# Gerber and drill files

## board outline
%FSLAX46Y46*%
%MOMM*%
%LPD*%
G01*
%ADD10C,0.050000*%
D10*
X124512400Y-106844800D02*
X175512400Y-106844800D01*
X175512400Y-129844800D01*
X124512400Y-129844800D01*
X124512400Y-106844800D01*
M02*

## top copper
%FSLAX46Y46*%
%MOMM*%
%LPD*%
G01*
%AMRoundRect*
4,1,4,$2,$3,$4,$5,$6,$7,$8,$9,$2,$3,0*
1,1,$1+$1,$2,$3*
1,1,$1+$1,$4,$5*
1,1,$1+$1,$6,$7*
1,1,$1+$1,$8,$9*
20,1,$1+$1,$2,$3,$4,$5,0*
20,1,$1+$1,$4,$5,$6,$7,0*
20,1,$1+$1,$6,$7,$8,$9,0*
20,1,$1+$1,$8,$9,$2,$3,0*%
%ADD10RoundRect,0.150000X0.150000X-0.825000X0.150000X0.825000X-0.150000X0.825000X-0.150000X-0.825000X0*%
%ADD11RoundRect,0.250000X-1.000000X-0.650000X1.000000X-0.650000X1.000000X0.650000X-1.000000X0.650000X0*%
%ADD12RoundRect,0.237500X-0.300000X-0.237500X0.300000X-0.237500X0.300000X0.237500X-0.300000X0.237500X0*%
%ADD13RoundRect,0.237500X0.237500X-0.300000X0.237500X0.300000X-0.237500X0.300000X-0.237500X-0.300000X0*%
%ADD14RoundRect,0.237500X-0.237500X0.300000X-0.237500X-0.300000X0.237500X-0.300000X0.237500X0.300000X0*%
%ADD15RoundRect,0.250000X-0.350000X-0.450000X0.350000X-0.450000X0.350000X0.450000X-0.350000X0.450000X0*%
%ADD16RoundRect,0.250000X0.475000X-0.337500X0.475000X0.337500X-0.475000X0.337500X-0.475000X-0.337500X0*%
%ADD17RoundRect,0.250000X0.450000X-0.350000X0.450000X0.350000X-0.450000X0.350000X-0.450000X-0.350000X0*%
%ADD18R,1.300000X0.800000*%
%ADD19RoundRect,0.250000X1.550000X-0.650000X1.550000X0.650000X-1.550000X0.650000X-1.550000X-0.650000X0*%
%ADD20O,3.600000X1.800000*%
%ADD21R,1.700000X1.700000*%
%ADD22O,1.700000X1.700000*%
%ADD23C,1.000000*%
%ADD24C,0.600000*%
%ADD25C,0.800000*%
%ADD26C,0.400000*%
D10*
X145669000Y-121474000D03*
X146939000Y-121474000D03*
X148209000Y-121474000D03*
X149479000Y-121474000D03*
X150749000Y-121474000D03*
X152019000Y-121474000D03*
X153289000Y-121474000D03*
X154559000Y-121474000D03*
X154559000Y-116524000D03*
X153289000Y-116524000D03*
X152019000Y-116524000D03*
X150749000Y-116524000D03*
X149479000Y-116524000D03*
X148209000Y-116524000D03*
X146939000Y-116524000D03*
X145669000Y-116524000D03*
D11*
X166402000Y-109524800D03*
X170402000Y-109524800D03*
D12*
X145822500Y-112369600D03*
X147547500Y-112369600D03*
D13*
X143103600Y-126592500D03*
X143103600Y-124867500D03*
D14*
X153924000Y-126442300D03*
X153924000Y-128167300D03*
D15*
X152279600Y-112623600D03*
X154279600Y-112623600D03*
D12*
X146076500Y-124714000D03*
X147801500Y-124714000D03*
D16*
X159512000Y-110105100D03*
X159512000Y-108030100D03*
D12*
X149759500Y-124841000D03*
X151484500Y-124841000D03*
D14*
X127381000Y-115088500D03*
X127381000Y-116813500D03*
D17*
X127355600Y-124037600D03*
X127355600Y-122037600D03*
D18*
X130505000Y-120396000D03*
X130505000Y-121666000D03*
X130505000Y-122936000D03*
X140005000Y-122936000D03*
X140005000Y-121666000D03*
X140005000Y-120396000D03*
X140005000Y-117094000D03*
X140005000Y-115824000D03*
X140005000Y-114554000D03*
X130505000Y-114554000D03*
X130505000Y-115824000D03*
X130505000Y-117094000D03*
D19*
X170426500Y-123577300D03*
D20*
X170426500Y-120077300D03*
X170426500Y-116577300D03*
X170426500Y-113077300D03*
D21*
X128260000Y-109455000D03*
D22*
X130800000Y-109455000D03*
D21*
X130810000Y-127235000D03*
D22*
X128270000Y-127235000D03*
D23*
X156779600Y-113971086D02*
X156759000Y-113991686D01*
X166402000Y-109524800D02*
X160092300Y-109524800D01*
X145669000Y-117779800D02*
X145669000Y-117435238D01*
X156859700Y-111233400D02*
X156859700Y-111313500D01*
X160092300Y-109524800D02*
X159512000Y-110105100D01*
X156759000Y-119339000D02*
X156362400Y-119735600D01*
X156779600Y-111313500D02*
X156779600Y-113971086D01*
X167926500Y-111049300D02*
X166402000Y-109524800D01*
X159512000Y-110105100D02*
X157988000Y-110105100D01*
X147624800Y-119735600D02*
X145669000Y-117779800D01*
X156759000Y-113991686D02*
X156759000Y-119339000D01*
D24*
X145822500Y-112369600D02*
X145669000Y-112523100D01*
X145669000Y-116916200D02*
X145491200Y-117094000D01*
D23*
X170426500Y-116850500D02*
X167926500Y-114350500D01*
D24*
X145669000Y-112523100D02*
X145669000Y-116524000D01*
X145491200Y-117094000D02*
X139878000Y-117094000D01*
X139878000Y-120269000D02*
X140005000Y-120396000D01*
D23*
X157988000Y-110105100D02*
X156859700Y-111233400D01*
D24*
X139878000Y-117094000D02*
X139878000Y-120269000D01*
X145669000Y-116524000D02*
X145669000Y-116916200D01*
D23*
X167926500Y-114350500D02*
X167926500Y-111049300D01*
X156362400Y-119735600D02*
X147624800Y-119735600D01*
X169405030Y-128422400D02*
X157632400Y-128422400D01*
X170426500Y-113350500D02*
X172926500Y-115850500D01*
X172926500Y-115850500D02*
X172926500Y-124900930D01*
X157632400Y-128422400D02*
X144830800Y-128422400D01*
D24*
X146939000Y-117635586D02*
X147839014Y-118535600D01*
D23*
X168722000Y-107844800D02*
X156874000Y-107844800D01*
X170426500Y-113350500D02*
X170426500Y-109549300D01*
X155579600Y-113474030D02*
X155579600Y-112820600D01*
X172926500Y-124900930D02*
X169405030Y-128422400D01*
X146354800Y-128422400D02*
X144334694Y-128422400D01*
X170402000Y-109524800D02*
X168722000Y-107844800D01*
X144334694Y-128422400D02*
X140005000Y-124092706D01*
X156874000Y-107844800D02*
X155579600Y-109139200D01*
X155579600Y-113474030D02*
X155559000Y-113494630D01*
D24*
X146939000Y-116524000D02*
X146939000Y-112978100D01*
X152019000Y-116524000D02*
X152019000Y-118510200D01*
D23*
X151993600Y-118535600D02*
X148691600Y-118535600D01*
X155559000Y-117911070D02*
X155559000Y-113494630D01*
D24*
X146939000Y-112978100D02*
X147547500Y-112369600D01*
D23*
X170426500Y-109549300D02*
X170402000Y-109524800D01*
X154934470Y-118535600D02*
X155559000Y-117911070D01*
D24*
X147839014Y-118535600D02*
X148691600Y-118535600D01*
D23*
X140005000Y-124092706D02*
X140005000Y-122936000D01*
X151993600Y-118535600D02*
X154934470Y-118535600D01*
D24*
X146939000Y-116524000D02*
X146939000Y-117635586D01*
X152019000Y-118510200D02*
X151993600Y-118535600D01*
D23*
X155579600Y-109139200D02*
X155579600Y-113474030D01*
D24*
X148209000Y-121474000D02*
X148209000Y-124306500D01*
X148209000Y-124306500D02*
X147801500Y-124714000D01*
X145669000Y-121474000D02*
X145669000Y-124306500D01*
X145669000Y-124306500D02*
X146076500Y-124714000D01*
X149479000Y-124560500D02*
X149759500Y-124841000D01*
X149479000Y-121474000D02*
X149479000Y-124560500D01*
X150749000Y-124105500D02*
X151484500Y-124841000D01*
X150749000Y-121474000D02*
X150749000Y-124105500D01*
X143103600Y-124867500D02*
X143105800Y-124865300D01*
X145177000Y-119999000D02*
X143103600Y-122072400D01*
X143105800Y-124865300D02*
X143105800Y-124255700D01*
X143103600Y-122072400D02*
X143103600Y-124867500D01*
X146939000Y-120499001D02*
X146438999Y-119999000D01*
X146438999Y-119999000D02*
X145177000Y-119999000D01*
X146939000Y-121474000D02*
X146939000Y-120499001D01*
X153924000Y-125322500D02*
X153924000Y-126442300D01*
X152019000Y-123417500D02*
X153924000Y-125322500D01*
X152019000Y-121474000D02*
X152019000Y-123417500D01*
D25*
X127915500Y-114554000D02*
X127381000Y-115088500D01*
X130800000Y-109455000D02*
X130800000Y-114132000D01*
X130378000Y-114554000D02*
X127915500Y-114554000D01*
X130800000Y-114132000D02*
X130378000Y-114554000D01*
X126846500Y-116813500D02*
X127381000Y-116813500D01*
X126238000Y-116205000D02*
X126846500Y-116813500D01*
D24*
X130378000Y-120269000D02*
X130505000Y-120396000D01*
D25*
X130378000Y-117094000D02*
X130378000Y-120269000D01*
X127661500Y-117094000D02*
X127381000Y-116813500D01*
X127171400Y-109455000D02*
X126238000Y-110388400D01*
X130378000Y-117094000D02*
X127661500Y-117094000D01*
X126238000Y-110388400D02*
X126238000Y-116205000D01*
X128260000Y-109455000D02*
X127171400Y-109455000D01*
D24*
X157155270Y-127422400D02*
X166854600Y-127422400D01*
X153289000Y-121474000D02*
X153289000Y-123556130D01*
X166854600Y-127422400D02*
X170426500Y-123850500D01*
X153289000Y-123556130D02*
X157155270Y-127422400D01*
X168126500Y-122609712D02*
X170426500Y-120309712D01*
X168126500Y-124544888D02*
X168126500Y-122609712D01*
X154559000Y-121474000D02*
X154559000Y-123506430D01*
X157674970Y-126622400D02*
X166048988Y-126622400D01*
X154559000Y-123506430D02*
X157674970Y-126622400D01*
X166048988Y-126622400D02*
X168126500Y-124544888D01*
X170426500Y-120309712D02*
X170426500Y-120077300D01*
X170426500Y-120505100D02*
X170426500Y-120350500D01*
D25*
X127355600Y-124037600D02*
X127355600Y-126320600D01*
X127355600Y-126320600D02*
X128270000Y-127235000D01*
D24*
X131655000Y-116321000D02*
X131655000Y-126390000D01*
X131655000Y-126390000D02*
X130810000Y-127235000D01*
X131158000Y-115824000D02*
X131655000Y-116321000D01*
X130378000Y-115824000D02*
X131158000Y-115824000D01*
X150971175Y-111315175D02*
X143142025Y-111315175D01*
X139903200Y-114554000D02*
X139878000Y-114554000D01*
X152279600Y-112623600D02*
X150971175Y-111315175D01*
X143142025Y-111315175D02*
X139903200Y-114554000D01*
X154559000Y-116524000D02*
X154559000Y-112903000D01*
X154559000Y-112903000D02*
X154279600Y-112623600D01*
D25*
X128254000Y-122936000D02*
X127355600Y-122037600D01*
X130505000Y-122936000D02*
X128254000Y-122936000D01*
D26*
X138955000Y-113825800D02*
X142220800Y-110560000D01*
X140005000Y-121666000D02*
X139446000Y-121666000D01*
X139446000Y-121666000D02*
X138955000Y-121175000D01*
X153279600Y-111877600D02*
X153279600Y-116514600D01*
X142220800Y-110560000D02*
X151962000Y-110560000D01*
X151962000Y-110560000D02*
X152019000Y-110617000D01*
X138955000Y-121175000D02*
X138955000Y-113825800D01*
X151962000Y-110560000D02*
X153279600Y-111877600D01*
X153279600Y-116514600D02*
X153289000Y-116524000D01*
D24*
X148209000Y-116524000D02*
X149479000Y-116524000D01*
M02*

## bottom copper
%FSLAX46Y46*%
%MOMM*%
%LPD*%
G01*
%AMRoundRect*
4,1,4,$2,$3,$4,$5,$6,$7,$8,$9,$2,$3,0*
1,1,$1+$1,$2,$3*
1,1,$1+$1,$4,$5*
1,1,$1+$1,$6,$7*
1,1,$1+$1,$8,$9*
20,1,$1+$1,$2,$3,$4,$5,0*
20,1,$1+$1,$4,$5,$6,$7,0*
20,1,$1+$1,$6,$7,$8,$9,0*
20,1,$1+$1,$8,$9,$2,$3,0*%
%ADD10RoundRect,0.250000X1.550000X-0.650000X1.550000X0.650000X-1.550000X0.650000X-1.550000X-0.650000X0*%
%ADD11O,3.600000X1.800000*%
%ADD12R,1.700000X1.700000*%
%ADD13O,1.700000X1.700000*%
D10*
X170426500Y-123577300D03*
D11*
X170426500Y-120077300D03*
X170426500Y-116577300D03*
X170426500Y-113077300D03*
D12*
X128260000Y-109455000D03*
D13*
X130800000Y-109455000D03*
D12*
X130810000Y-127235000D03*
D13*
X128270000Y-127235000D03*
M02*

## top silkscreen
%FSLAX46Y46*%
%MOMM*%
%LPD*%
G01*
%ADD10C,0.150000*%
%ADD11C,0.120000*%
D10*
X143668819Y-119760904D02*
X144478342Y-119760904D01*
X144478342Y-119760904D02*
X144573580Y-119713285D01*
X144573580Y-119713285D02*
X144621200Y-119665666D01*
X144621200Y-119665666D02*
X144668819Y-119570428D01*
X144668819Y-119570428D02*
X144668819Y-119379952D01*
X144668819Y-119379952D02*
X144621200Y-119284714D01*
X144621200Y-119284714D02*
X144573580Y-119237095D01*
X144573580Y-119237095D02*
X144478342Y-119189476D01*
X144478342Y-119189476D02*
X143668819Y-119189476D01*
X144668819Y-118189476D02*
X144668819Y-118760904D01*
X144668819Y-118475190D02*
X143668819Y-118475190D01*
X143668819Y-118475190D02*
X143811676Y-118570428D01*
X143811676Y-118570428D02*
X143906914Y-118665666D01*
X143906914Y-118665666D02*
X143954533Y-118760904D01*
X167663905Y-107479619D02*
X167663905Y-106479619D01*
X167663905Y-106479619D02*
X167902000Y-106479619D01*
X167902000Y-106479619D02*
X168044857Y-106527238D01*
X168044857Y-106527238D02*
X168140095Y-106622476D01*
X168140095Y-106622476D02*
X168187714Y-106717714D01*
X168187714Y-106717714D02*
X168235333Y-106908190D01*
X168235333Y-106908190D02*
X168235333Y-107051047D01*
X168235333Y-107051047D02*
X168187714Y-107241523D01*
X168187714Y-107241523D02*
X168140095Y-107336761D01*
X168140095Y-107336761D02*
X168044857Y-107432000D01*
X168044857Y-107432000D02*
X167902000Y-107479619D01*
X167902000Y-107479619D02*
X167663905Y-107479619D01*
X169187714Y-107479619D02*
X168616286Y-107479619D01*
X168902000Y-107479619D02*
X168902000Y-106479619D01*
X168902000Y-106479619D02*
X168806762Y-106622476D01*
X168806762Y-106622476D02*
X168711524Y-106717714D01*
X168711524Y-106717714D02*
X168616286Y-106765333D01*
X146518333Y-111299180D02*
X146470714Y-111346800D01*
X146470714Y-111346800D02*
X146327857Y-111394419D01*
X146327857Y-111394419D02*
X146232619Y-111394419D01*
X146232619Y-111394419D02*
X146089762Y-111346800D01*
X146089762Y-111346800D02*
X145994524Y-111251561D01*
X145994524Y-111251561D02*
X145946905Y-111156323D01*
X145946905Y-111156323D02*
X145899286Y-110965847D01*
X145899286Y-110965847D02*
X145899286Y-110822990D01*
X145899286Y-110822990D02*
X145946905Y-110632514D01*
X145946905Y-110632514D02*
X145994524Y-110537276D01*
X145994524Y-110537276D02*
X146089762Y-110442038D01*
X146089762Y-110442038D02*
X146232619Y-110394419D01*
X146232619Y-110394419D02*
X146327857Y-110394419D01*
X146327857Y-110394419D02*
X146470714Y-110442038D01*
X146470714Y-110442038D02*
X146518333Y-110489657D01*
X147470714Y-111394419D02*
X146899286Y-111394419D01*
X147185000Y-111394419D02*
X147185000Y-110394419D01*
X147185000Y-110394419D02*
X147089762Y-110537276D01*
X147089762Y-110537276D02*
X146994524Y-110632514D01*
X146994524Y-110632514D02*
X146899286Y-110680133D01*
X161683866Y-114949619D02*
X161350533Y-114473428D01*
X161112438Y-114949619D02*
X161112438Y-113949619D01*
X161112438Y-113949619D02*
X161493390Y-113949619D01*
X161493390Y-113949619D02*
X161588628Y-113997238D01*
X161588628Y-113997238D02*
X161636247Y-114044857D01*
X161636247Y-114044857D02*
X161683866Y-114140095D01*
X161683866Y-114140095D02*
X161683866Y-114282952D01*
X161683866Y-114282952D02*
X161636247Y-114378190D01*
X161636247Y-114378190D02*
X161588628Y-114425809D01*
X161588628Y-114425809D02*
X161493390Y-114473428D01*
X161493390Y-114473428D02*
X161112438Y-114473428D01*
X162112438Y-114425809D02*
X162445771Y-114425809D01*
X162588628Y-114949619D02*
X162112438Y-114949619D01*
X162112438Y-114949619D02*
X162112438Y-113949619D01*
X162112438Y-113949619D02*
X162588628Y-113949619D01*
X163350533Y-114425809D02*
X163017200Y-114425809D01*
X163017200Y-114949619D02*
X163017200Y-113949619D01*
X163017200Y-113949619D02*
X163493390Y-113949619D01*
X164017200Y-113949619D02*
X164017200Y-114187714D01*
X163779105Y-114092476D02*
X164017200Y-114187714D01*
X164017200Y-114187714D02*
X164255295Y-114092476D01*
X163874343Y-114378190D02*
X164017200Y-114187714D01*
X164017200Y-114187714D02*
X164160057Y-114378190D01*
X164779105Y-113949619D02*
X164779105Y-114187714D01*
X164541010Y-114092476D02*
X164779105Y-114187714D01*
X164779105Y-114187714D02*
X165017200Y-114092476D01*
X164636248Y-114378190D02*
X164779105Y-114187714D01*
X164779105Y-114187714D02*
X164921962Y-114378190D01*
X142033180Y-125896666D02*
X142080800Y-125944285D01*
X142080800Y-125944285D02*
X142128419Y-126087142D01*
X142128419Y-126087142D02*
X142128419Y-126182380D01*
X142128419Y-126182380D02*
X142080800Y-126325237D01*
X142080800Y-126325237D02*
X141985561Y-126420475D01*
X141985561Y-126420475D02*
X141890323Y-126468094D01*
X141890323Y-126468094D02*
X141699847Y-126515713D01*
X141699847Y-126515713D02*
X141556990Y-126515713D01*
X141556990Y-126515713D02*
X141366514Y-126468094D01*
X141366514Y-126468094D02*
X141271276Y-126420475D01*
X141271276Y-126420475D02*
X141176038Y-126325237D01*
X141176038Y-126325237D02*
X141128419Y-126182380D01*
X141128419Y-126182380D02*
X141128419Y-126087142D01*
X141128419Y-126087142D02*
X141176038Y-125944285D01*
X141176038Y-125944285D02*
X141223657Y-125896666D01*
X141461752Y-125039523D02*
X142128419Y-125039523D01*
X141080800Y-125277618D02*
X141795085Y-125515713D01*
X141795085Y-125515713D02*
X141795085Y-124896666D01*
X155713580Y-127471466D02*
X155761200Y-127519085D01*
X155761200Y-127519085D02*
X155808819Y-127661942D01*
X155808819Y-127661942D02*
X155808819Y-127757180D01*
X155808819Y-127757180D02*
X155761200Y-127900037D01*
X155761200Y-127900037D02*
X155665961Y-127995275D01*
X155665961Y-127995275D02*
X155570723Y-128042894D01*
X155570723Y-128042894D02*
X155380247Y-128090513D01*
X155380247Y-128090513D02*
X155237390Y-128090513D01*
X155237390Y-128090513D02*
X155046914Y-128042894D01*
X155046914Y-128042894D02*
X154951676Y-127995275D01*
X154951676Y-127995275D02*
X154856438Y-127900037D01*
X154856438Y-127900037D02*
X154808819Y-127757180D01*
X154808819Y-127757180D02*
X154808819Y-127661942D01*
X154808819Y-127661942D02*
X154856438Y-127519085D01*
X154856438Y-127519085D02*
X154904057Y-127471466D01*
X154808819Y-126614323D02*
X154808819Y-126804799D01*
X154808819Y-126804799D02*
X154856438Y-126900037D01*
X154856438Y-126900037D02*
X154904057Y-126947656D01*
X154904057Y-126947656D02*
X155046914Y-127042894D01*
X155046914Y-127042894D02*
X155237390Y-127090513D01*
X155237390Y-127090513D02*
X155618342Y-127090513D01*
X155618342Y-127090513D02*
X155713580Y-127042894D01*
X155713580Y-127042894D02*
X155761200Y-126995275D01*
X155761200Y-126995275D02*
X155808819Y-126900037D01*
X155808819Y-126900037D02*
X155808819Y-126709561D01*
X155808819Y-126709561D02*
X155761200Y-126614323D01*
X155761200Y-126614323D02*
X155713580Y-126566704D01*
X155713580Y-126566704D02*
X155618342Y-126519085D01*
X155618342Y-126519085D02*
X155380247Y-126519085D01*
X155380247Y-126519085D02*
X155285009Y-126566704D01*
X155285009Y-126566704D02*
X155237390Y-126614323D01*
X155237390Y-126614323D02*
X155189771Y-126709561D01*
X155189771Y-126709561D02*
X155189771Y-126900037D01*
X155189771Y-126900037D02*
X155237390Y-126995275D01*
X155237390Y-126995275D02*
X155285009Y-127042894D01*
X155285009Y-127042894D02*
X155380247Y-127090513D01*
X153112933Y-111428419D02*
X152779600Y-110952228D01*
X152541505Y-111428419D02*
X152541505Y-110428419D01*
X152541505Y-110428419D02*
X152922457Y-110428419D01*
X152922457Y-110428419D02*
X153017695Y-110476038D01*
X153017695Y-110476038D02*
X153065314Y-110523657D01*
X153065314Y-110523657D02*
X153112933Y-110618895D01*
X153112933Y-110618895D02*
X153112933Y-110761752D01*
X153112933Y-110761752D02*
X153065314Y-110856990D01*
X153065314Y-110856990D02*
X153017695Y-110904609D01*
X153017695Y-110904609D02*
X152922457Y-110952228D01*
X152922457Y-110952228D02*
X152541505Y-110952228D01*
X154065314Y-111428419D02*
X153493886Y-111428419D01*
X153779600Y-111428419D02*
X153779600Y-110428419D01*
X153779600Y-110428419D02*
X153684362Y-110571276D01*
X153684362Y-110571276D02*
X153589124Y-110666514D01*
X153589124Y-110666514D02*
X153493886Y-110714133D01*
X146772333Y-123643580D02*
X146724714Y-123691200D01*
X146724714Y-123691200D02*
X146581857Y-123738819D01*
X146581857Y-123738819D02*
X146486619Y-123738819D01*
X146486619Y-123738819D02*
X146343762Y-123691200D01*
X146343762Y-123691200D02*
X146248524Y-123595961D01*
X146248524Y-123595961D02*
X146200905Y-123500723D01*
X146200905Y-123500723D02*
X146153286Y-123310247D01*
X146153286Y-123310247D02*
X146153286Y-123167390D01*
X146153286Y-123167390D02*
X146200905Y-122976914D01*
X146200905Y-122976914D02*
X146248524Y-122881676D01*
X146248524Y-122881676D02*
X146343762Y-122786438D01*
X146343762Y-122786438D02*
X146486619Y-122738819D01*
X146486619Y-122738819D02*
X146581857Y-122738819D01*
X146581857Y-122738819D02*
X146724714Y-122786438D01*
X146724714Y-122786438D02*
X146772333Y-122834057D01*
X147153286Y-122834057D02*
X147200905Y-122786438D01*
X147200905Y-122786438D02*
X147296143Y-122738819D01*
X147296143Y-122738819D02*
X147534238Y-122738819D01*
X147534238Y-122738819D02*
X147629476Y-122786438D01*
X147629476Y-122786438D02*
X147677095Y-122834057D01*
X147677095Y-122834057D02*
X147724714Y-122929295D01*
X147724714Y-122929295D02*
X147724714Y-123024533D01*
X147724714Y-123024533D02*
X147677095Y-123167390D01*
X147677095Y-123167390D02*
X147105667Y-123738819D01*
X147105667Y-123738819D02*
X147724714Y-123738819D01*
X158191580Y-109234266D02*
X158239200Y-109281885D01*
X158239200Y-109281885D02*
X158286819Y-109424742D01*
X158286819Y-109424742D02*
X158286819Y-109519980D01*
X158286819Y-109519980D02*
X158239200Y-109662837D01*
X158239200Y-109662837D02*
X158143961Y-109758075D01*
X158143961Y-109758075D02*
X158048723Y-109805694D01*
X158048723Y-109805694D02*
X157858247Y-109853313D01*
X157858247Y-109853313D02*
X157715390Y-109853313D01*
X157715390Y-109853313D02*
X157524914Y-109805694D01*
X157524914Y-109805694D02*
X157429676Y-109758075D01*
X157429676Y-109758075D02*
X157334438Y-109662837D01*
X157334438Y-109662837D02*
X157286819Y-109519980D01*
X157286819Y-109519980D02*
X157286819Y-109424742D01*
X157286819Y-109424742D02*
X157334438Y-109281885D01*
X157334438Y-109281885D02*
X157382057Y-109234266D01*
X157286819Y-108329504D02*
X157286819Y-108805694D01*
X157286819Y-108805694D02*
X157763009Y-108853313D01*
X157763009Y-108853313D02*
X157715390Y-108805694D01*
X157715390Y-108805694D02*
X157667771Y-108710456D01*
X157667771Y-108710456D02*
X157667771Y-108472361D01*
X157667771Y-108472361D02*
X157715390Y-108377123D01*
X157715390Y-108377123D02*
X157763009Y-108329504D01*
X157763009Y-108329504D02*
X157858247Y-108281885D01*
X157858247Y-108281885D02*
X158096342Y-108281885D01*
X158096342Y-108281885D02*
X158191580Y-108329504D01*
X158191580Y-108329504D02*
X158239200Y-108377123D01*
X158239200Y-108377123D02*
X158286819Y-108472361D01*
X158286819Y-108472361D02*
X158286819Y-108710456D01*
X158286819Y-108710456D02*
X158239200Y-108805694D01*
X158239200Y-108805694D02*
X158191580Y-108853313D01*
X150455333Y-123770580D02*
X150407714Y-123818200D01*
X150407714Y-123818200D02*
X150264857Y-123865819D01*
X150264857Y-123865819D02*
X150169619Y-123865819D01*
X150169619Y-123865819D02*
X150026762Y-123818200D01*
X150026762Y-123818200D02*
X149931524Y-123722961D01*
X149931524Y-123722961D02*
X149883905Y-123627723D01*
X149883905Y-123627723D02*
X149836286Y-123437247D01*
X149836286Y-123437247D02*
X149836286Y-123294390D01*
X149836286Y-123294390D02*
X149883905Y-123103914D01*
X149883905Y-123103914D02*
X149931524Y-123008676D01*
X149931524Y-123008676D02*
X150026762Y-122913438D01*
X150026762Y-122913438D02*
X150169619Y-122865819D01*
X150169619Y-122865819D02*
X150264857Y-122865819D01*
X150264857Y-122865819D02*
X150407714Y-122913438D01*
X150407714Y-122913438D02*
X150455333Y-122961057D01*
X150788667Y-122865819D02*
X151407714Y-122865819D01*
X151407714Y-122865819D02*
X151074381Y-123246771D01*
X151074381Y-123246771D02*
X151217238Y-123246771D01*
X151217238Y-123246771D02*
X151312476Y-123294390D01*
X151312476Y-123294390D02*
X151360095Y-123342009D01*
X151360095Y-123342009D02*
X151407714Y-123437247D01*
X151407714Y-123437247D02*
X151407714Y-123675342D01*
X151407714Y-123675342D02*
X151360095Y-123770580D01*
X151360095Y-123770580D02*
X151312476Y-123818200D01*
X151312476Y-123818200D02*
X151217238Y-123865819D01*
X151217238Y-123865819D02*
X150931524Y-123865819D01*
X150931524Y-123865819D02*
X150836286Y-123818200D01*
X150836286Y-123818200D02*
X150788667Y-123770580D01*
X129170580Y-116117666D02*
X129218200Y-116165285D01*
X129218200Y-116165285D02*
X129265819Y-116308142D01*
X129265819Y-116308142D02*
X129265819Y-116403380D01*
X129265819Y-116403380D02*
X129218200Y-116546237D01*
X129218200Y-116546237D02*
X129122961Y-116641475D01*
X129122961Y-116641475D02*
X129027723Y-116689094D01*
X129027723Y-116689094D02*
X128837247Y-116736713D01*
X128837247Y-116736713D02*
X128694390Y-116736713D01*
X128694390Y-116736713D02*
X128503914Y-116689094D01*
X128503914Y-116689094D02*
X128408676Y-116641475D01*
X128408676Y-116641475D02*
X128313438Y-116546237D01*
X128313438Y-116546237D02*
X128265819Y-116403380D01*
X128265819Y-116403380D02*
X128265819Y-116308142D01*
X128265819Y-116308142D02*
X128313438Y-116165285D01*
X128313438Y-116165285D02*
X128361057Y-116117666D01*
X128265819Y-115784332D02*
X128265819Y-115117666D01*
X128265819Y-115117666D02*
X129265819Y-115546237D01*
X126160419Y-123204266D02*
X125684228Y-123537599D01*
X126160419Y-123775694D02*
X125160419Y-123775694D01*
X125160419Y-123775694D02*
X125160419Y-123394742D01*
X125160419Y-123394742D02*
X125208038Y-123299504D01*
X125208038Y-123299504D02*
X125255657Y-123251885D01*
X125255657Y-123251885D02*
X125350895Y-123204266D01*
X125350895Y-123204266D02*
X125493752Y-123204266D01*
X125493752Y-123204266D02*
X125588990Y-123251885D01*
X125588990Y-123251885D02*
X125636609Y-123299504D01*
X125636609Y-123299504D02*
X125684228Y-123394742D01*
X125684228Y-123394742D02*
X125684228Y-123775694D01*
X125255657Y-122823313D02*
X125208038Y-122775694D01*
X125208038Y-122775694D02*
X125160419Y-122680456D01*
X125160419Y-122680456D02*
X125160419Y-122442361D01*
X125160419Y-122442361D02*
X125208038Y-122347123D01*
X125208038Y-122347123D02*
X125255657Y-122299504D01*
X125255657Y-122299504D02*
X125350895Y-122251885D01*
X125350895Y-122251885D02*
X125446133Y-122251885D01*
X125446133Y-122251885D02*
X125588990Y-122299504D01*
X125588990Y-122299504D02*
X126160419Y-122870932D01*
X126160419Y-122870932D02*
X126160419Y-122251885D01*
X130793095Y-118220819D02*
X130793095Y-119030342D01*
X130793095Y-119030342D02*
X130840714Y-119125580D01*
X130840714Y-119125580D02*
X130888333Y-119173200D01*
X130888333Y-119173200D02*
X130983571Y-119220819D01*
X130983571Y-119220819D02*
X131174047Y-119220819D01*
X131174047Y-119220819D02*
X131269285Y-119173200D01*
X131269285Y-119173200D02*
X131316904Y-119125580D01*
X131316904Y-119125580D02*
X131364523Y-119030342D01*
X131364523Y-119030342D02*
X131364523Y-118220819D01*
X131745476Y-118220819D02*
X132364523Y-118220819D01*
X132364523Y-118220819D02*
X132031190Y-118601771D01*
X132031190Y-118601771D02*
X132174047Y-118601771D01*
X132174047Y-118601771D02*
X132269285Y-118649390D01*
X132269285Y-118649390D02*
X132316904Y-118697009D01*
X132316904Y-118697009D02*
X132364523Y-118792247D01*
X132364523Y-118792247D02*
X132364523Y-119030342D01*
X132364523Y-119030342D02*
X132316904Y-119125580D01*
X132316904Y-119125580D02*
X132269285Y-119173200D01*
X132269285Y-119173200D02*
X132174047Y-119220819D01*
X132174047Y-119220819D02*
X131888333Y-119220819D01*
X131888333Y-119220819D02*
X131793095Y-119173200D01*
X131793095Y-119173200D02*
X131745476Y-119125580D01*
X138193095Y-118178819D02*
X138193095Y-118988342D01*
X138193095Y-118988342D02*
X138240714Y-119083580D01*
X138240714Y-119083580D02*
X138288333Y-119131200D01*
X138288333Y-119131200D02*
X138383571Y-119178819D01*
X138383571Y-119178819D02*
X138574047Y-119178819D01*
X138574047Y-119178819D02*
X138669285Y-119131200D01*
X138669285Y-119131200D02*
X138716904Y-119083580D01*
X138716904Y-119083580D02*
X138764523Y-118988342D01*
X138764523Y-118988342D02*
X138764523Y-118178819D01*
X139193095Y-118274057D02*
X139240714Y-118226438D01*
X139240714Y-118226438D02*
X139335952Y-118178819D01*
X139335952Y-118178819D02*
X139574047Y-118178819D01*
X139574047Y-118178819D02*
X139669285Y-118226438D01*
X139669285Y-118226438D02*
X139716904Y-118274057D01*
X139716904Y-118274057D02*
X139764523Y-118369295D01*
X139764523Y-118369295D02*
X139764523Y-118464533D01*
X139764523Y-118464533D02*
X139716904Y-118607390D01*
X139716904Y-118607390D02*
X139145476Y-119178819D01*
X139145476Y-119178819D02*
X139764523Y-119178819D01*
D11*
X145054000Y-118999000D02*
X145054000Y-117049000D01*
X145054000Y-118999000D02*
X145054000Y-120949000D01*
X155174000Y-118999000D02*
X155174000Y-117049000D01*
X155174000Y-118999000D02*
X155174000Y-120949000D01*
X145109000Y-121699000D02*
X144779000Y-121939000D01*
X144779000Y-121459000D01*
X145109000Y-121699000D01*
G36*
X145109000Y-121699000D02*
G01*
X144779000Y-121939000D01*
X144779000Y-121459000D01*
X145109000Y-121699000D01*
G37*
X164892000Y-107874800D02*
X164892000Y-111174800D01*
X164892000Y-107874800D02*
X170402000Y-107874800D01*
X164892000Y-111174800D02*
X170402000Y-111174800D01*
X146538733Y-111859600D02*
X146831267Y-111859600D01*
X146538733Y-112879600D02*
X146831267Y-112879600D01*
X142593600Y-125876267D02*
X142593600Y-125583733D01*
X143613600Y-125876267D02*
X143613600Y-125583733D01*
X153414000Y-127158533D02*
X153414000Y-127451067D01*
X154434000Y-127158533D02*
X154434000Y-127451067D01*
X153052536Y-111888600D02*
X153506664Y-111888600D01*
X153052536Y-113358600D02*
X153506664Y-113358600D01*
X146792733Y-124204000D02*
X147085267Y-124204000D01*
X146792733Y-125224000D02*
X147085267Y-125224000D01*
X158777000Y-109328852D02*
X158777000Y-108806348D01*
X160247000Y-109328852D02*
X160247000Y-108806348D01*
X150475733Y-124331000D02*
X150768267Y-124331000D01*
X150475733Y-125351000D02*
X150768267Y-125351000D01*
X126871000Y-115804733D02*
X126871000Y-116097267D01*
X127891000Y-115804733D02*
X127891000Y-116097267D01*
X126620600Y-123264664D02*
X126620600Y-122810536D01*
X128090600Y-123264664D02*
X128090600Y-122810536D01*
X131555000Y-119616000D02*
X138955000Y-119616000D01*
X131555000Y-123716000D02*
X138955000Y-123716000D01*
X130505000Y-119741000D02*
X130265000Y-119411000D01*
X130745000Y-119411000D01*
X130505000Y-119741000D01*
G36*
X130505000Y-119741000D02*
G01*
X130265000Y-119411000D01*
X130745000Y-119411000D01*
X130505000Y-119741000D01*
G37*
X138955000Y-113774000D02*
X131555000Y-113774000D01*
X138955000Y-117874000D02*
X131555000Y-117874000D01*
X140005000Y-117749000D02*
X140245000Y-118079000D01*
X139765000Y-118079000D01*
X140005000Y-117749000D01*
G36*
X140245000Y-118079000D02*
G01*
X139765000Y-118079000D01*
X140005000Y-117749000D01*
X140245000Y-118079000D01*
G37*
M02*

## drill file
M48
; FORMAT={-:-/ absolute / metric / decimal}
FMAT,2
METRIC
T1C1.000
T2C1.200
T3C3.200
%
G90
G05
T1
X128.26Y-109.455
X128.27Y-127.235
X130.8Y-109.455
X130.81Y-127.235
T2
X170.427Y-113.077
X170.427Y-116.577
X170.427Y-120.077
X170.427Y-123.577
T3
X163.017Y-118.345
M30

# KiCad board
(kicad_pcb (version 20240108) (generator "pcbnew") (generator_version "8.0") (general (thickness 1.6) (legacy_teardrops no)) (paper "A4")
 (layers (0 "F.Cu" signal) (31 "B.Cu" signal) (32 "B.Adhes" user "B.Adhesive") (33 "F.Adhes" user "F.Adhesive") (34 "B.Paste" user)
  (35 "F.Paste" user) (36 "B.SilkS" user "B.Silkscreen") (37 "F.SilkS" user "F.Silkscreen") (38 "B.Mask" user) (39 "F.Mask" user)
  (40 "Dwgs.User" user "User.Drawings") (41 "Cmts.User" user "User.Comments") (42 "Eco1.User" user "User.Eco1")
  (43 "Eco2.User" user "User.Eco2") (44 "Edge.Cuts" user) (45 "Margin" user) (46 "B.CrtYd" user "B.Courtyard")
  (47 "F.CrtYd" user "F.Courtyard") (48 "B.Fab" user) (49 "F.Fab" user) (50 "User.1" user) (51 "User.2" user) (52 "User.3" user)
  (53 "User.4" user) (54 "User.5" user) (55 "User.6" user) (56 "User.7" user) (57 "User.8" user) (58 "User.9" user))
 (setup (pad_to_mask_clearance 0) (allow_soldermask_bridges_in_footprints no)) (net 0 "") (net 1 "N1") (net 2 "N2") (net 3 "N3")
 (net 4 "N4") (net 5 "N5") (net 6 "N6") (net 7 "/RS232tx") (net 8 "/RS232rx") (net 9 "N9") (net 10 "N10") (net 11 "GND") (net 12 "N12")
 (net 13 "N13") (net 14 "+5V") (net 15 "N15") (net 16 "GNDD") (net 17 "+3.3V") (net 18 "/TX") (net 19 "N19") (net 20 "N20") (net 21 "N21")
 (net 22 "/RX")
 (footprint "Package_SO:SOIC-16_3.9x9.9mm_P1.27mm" (layer "F.Cu") (at 150.114 118.999 90)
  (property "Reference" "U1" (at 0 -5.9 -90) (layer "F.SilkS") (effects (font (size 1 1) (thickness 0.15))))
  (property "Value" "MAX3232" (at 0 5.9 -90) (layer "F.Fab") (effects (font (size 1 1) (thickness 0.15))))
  (fp_line (start 0 -5.06) (end 1.95 -5.06) (stroke (width 0.12) (type solid)) (layer "F.SilkS"))
  (fp_line (start 0 -5.06) (end -1.95 -5.06) (stroke (width 0.12) (type solid)) (layer "F.SilkS"))
  (fp_line (start 0 5.06) (end 1.95 5.06) (stroke (width 0.12) (type solid)) (layer "F.SilkS"))
  (fp_line (start 0 5.06) (end -1.95 5.06) (stroke (width 0.12) (type solid)) (layer "F.SilkS"))
  (fp_poly
   (pts (xy -2.7 -5.005) (xy -2.94 -5.335) (xy -2.46 -5.335) (xy -2.7 -5.005)) (stroke (width 0.12) (type solid)) (fill solid)
   (layer "F.SilkS"))
  (pad "1" smd roundrect (at -2.475 -4.445 90) (size 1.95 0.6) (layers "F.Cu" "F.Paste" "F.Mask") (roundrect_rratio 0.25) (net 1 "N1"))
  (pad "2" smd roundrect (at -2.475 -3.175 90) (size 1.95 0.6) (layers "F.Cu" "F.Paste" "F.Mask") (roundrect_rratio 0.25) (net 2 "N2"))
  (pad "3" smd roundrect (at -2.475 -1.905 90) (size 1.95 0.6) (layers "F.Cu" "F.Paste" "F.Mask") (roundrect_rratio 0.25) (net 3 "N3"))
  (pad "4" smd roundrect (at -2.475 -0.635 90) (size 1.95 0.6) (layers "F.Cu" "F.Paste" "F.Mask") (roundrect_rratio 0.25) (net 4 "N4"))
  (pad "5" smd roundrect (at -2.475 0.635 90) (size 1.95 0.6) (layers "F.Cu" "F.Paste" "F.Mask") (roundrect_rratio 0.25) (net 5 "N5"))
  (pad "6" smd roundrect (at -2.475 1.905 90) (size 1.95 0.6) (layers "F.Cu" "F.Paste" "F.Mask") (roundrect_rratio 0.25) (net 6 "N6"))
  (pad "7" smd roundrect (at -2.475 3.175 90) (size 1.95 0.6) (layers "F.Cu" "F.Paste" "F.Mask") (roundrect_rratio 0.25) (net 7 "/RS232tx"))
  (pad "8" smd roundrect (at -2.475 4.445 90) (size 1.95 0.6) (layers "F.Cu" "F.Paste" "F.Mask") (roundrect_rratio 0.25) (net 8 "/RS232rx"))
  (pad "9" smd roundrect (at 2.475 4.445 90) (size 1.95 0.6) (layers "F.Cu" "F.Paste" "F.Mask") (roundrect_rratio 0.25) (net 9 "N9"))
  (pad "10" smd roundrect (at 2.475 3.175 90) (size 1.95 0.6) (layers "F.Cu" "F.Paste" "F.Mask") (roundrect_rratio 0.25) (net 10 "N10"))
  (pad "11" smd roundrect (at 2.475 1.905 90) (size 1.95 0.6) (layers "F.Cu" "F.Paste" "F.Mask") (roundrect_rratio 0.25) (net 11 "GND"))
  (pad "12" smd roundrect (at 2.475 0.635 90) (size 1.95 0.6) (layers "F.Cu" "F.Paste" "F.Mask") (roundrect_rratio 0.25) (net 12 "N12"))
  (pad "13" smd roundrect (at 2.475 -0.635 90) (size 1.95 0.6) (layers "F.Cu" "F.Paste" "F.Mask") (roundrect_rratio 0.25) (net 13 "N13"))
  (pad "14" smd roundrect (at 2.475 -1.905 90) (size 1.95 0.6) (layers "F.Cu" "F.Paste" "F.Mask") (roundrect_rratio 0.25) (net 13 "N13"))
  (pad "15" smd roundrect (at 2.475 -3.175 90) (size 1.95 0.6) (layers "F.Cu" "F.Paste" "F.Mask") (roundrect_rratio 0.25) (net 11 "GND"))
  (pad "16" smd roundrect (at 2.475 -4.445 90) (size 1.95 0.6) (layers "F.Cu" "F.Paste" "F.Mask") (roundrect_rratio 0.25) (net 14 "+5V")))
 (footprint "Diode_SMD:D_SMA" (layer "F.Cu") (at 168.402 109.5248)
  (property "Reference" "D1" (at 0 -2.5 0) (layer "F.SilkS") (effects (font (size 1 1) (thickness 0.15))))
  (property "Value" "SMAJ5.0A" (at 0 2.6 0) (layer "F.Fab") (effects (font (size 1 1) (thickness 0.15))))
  (fp_line (start -3.51 -1.65) (end -3.51 1.65) (stroke (width 0.12) (type solid)) (layer "F.SilkS"))
  (fp_line (start -3.51 -1.65) (end 2 -1.65) (stroke (width 0.12) (type solid)) (layer "F.SilkS"))
  (fp_line (start -3.51 1.65) (end 2 1.65) (stroke (width 0.12) (type solid)) (layer "F.SilkS"))
  (pad "1" smd roundrect (at -2 0) (size 2.5 1.8) (layers "F.Cu" "F.Paste" "F.Mask") (roundrect_rratio 0.1388888889) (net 14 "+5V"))
  (pad "2" smd roundrect (at 2 0) (size 2.5 1.8) (layers "F.Cu" "F.Paste" "F.Mask") (roundrect_rratio 0.1388888889) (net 11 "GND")))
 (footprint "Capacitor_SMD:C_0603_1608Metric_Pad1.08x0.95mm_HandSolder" (layer "F.Cu") (at 146.685 112.3696)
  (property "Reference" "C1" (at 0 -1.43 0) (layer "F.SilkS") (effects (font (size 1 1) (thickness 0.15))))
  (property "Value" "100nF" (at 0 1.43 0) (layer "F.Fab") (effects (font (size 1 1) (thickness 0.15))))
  (fp_line (start -0.146267 -0.51) (end 0.146267 -0.51) (stroke (width 0.12) (type solid)) (layer "F.SilkS"))
  (fp_line (start -0.146267 0.51) (end 0.146267 0.51) (stroke (width 0.12) (type solid)) (layer "F.SilkS"))
  (pad "1" smd roundrect (at -0.8625 0) (size 1.075 0.95) (layers "F.Cu" "F.Paste" "F.Mask") (roundrect_rratio 0.25) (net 14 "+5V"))
  (pad "2" smd roundrect (at 0.8625 0) (size 1.075 0.95) (layers "F.Cu" "F.Paste" "F.Mask") (roundrect_rratio 0.25) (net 11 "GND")))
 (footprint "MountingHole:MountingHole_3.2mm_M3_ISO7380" (layer "F.Cu") (at 163.0172 118.3448)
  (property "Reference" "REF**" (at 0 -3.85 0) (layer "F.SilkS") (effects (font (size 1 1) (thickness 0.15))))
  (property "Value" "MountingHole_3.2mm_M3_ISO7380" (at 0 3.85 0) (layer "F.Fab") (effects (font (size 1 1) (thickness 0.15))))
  (pad "" np_thru_hole circle (at 0 0) (size 3.2 3.2) (drill 3.2) (layers "F&B.Cu" "*.Mask") (clearance 4)))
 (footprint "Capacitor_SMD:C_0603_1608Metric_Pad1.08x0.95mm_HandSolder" (layer "F.Cu") (at 143.1036 125.73 90)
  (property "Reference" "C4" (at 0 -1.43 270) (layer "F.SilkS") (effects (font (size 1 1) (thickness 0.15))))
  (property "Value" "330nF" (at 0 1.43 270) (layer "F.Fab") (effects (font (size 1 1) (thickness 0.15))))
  (fp_line (start -0.146267 -0.51) (end 0.146267 -0.51) (stroke (width 0.12) (type solid)) (layer "F.SilkS"))
  (fp_line (start -0.146267 0.51) (end 0.146267 0.51) (stroke (width 0.12) (type solid)) (layer "F.SilkS"))
  (pad "1" smd roundrect (at -0.8625 0 90) (size 1.075 0.95) (layers "F.Cu" "F.Paste" "F.Mask") (roundrect_rratio 0.25) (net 11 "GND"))
  (pad "2" smd roundrect (at 0.8625 0 90) (size 1.075 0.95) (layers "F.Cu" "F.Paste" "F.Mask") (roundrect_rratio 0.25) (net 2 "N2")))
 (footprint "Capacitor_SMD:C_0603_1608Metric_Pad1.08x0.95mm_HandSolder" (layer "F.Cu") (at 153.924 127.3048 -90)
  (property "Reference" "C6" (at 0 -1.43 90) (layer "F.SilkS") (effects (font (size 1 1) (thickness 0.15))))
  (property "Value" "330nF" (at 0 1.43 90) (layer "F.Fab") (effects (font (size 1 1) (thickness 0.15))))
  (fp_line (start -0.146267 0.51) (end 0.146267 0.51) (stroke (width 0.12) (type solid)) (layer "F.SilkS"))
  (fp_line (start -0.146267 -0.51) (end 0.146267 -0.51) (stroke (width 0.12) (type solid)) (layer "F.SilkS"))
  (pad "1" smd roundrect (at -0.8625 0 270) (size 1.075 0.95) (layers "F.Cu" "F.Paste" "F.Mask") (roundrect_rratio 0.25) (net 6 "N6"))
  (pad "2" smd roundrect (at 0.8625 0 270) (size 1.075 0.95) (layers "F.Cu" "F.Paste" "F.Mask") (roundrect_rratio 0.25) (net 11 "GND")))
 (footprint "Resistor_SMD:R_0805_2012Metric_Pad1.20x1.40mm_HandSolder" (layer "F.Cu") (at 153.2796 112.6236)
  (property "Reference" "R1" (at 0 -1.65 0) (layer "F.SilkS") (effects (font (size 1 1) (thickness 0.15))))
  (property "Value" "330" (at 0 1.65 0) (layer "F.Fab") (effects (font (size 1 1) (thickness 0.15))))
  (fp_line (start -0.227064 -0.735) (end 0.227064 -0.735) (stroke (width 0.12) (type solid)) (layer "F.SilkS"))
  (fp_line (start -0.227064 0.735) (end 0.227064 0.735) (stroke (width 0.12) (type solid)) (layer "F.SilkS"))
  (pad "1" smd roundrect (at -1 0) (size 1.2 1.4) (layers "F.Cu" "F.Paste" "F.Mask") (roundrect_rratio 0.208333) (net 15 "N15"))
  (pad "2" smd roundrect (at 1 0) (size 1.2 1.4) (layers "F.Cu" "F.Paste" "F.Mask") (roundrect_rratio 0.208333) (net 9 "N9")))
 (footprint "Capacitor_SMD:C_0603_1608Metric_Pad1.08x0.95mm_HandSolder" (layer "F.Cu") (at 146.939 124.714)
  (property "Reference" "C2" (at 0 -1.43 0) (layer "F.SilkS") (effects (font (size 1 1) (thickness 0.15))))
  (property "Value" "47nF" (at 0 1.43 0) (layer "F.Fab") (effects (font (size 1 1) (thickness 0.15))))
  (fp_line (start -0.146267 -0.51) (end 0.146267 -0.51) (stroke (width 0.12) (type solid)) (layer "F.SilkS"))
  (fp_line (start -0.146267 0.51) (end 0.146267 0.51) (stroke (width 0.12) (type solid)) (layer "F.SilkS"))
  (pad "1" smd roundrect (at -0.8625 0) (size 1.075 0.95) (layers "F.Cu" "F.Paste" "F.Mask") (roundrect_rratio 0.25) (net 1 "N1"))
  (pad "2" smd roundrect (at 0.8625 0) (size 1.075 0.95) (layers "F.Cu" "F.Paste" "F.Mask") (roundrect_rratio 0.25) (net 3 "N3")))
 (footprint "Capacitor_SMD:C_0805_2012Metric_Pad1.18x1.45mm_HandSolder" (layer "F.Cu") (at 159.512 109.0676 90)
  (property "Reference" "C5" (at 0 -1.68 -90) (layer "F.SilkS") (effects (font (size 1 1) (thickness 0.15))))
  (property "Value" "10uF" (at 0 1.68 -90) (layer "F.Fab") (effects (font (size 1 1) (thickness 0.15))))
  (fp_line (start -0.261252 -0.735) (end 0.261252 -0.735) (stroke (width 0.12) (type solid)) (layer "F.SilkS"))
  (fp_line (start -0.261252 0.735) (end 0.261252 0.735) (stroke (width 0.12) (type solid)) (layer "F.SilkS"))
  (pad "1" smd roundrect (at -1.0375 0 90) (size 1.175 1.45) (layers "F.Cu" "F.Paste" "F.Mask") (roundrect_rratio 0.212766) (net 14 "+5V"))
  (pad "2" smd roundrect (at 1.0375 0 90) (size 1.175 1.45) (layers "F.Cu" "F.Paste" "F.Mask") (roundrect_rratio 0.212766) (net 11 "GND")))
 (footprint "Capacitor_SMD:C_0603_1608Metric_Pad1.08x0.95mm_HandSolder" (layer "F.Cu") (at 150.622 124.841)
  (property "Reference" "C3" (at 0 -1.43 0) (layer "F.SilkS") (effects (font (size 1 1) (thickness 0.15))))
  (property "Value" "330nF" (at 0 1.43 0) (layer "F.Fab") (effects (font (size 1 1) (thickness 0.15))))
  (fp_line (start -0.146267 -0.51) (end 0.146267 -0.51) (stroke (width 0.12) (type solid)) (layer "F.SilkS"))
  (fp_line (start -0.146267 0.51) (end 0.146267 0.51) (stroke (width 0.12) (type solid)) (layer "F.SilkS"))
  (pad "1" smd roundrect (at -0.8625 0) (size 1.075 0.95) (layers "F.Cu" "F.Paste" "F.Mask") (roundrect_rratio 0.25) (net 4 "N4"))
  (pad "2" smd roundrect (at 0.8625 0) (size 1.075 0.95) (layers "F.Cu" "F.Paste" "F.Mask") (roundrect_rratio 0.25) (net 5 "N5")))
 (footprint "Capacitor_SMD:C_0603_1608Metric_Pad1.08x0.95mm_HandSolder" (layer "F.Cu") (at 127.381 115.951 -90)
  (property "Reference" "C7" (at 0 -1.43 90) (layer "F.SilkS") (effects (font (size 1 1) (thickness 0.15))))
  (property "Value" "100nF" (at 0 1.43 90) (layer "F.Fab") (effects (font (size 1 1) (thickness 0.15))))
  (fp_line (start -0.146267 0.51) (end 0.146267 0.51) (stroke (width 0.12) (type solid)) (layer "F.SilkS"))
  (fp_line (start -0.146267 -0.51) (end 0.146267 -0.51) (stroke (width 0.12) (type solid)) (layer "F.SilkS"))
  (pad "1" smd roundrect (at -0.8625 0 270) (size 1.075 0.95) (layers "F.Cu" "F.Paste" "F.Mask") (roundrect_rratio 0.25) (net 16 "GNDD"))
  (pad "2" smd roundrect (at 0.8625 0 270) (size 1.075 0.95) (layers "F.Cu" "F.Paste" "F.Mask") (roundrect_rratio 0.25) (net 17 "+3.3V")))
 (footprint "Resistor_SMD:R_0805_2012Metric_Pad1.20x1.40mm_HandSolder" (layer "F.Cu") (at 127.3556 123.0376 90)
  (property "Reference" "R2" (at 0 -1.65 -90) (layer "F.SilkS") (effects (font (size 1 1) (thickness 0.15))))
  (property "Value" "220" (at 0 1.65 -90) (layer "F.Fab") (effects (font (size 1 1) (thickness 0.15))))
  (fp_line (start -0.227064 -0.735) (end 0.227064 -0.735) (stroke (width 0.12) (type solid)) (layer "F.SilkS"))
  (fp_line (start -0.227064 0.735) (end 0.227064 0.735) (stroke (width 0.12) (type solid)) (layer "F.SilkS"))
  (pad "1" smd roundrect (at -1 0 90) (size 1.2 1.4) (layers "F.Cu" "F.Paste" "F.Mask") (roundrect_rratio 0.208333) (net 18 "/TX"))
  (pad "2" smd roundrect (at 1 0 90) (size 1.2 1.4) (layers "F.Cu" "F.Paste" "F.Mask") (roundrect_rratio 0.208333) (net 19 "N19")))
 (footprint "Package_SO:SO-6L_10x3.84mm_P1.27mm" (layer "F.Cu") (at 135.255 121.666)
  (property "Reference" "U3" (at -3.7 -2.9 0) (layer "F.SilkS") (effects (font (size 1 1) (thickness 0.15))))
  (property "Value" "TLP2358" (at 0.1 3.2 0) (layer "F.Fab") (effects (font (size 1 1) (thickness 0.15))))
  (fp_line (start -3.7 -2.05) (end 3.7 -2.05) (stroke (width 0.12) (type solid)) (layer "F.SilkS"))
  (fp_line (start -3.7 2.05) (end 3.7 2.05) (stroke (width 0.12) (type solid)) (layer "F.SilkS"))
  (fp_poly
   (pts (xy -4.75 -1.925) (xy -4.99 -2.255) (xy -4.51 -2.255) (xy -4.75 -1.925)) (stroke (width 0.12) (type solid)) (fill solid)
   (layer "F.SilkS"))
  (pad "1" smd rect (at -4.75 -1.27 90) (size 0.8 1.3) (layers "F.Cu" "F.Paste" "F.Mask") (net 17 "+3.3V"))
  (pad "2" smd rect (at -4.75 0 90) (size 0.8 1.3) (layers "F.Cu" "F.Paste" "F.Mask") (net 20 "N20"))
  (pad "3" smd rect (at -4.75 1.27 90) (size 0.8 1.3) (layers "F.Cu" "F.Paste" "F.Mask") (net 19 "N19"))
  (pad "4" smd rect (at 4.75 1.27 90) (size 0.8 1.3) (layers "F.Cu" "F.Paste" "F.Mask") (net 11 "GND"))
  (pad "5" smd rect (at 4.75 0 90) (size 0.8 1.3) (layers "F.Cu" "F.Paste" "F.Mask") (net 10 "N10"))
  (pad "6" smd rect (at 4.75 -1.27 90) (size 0.8 1.3) (layers "F.Cu" "F.Paste" "F.Mask") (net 14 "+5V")))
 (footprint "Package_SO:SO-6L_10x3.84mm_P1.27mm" (layer "F.Cu") (at 135.255 115.824 180)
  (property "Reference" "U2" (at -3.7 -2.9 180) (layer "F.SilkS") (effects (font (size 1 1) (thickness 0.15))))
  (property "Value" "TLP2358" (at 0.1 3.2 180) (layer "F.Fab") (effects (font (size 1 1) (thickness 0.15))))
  (fp_line (start -3.7 2.05) (end 3.7 2.05) (stroke (width 0.12) (type solid)) (layer "F.SilkS"))
  (fp_line (start -3.7 -2.05) (end 3.7 -2.05) (stroke (width 0.12) (type solid)) (layer "F.SilkS"))
  (fp_poly
   (pts (xy -4.75 -1.925) (xy -4.99 -2.255) (xy -4.51 -2.255) (xy -4.75 -1.925)) (stroke (width 0.12) (type solid)) (fill solid)
   (layer "F.SilkS"))
  (pad "1" smd rect (at -4.75 -1.27 270) (size 0.8 1.3) (layers "F.Cu" "F.Paste" "F.Mask") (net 14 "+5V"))
  (pad "2" smd rect (at -4.75 0 270) (size 0.8 1.3) (layers "F.Cu" "F.Paste" "F.Mask") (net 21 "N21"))
  (pad "3" smd rect (at -4.75 1.27 270) (size 0.8 1.3) (layers "F.Cu" "F.Paste" "F.Mask") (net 15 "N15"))
  (pad "4" smd rect (at 4.75 1.27 270) (size 0.8 1.3) (layers "F.Cu" "F.Paste" "F.Mask") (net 16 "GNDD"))
  (pad "5" smd rect (at 4.75 0 270) (size 0.8 1.3) (layers "F.Cu" "F.Paste" "F.Mask") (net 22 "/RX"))
  (pad "6" smd rect (at 4.75 -1.27 270) (size 0.8 1.3) (layers "F.Cu" "F.Paste" "F.Mask") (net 17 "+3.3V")))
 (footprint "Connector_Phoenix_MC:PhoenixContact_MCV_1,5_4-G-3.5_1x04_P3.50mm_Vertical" (layer "B.Cu") (at 170.4265 123.5773 90)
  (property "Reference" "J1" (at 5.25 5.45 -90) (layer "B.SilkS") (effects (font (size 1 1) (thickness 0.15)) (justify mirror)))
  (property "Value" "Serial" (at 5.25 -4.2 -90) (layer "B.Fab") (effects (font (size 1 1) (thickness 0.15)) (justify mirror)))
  (pad "1" thru_hole roundrect (at 0 0 90) (size 1.8 3.6) (drill 1.2) (layers "*.Cu" "*.Mask") (remove_unused_layers no)
   (roundrect_rratio 0.138889) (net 7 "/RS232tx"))
  (pad "2" thru_hole oval (at 3.5 0 90) (size 1.8 3.6) (drill 1.2) (layers "*.Cu" "*.Mask") (remove_unused_layers no) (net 8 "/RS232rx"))
  (pad "3" thru_hole oval (at 7 0 90) (size 1.8 3.6) (drill 1.2) (layers "*.Cu" "*.Mask") (remove_unused_layers no) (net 14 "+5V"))
  (pad "4" thru_hole oval (at 10.5 0 90) (size 1.8 3.6) (drill 1.2) (layers "*.Cu" "*.Mask") (remove_unused_layers no) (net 11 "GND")))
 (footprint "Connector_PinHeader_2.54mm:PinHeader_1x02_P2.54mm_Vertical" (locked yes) (layer "B.Cu") (at 128.26 109.455 -90)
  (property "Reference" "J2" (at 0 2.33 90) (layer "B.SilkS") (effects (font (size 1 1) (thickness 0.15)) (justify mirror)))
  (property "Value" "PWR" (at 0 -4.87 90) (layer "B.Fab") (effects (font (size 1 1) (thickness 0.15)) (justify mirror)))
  (pad "1" thru_hole rect (at 0 0 270) (size 1.7 1.7) (drill 1) (layers "*.Cu" "*.Mask") (remove_unused_layers no) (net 17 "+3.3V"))
  (pad "2" thru_hole oval (at 0 -2.54 270) (size 1.7 1.7) (drill 1) (layers "*.Cu" "*.Mask") (remove_unused_layers no) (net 16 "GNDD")))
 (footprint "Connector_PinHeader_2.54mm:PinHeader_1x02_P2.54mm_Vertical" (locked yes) (layer "B.Cu") (at 130.81 127.235 90)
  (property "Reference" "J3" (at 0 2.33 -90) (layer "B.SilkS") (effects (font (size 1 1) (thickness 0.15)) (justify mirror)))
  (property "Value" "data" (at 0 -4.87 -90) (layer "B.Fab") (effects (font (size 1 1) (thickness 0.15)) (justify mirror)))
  (pad "1" thru_hole rect (at 0 0 90) (size 1.7 1.7) (drill 1) (layers "*.Cu" "*.Mask") (remove_unused_layers no) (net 22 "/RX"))
  (pad "2" thru_hole oval (at 0 -2.54 90) (size 1.7 1.7) (drill 1) (layers "*.Cu" "*.Mask") (remove_unused_layers no) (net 18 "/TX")))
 (gr_rect (start 124.5124 106.8448) (end 175.5124 129.8448) (stroke (width 0.05) (type default)) (fill none) (layer "Edge.Cuts"))
 (segment (start 156.7796 113.971086) (end 156.759 113.991686) (width 1) (layer "F.Cu") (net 14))
 (segment (start 166.402 109.5248) (end 160.0923 109.5248) (width 1) (layer "F.Cu") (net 14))
 (segment (start 145.669 117.7798) (end 145.669 117.435238) (width 1) (layer "F.Cu") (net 14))
 (segment (start 156.8597 111.2334) (end 156.8597 111.3135) (width 1) (layer "F.Cu") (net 14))
 (segment (start 160.0923 109.5248) (end 159.512 110.1051) (width 1) (layer "F.Cu") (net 14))
 (segment (start 156.759 119.339) (end 156.3624 119.7356) (width 1) (layer "F.Cu") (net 14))
 (segment (start 156.7796 111.3135) (end 156.7796 113.971086) (width 1) (layer "F.Cu") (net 14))
 (segment (start 167.9265 111.0493) (end 166.402 109.5248) (width 1) (layer "F.Cu") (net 14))
 (segment (start 159.512 110.1051) (end 157.988 110.1051) (width 1) (layer "F.Cu") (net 14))
 (segment (start 147.6248 119.7356) (end 145.669 117.7798) (width 1) (layer "F.Cu") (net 14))
 (segment (start 156.759 113.991686) (end 156.759 119.339) (width 1) (layer "F.Cu") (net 14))
 (segment (start 145.8225 112.3696) (end 145.669 112.5231) (width 0.6) (layer "F.Cu") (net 14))
 (segment (start 145.669 116.9162) (end 145.4912 117.094) (width 0.6) (layer "F.Cu") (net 14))
 (segment (start 170.4265 116.8505) (end 167.9265 114.3505) (width 1) (layer "F.Cu") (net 14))
 (segment (start 145.669 112.5231) (end 145.669 116.524) (width 0.6) (layer "F.Cu") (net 14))
 (segment (start 145.4912 117.094) (end 139.878 117.094) (width 0.6) (layer "F.Cu") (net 14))
 (segment (start 139.878 120.269) (end 140.005 120.396) (width 0.6) (layer "F.Cu") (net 14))
 (segment (start 157.988 110.1051) (end 156.8597 111.2334) (width 1) (layer "F.Cu") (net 14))
 (segment (start 139.878 117.094) (end 139.878 120.269) (width 0.6) (layer "F.Cu") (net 14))
 (segment (start 145.669 116.524) (end 145.669 116.9162) (width 0.6) (layer "F.Cu") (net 14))
 (segment (start 167.9265 114.3505) (end 167.9265 111.0493) (width 1) (layer "F.Cu") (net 14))
 (segment (start 156.3624 119.7356) (end 147.6248 119.7356) (width 1) (layer "F.Cu") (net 14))
 (segment (start 169.40503 128.4224) (end 157.6324 128.4224) (width 1) (layer "F.Cu") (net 11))
 (segment (start 170.4265 113.3505) (end 172.9265 115.8505) (width 1) (layer "F.Cu") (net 11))
 (segment (start 172.9265 115.8505) (end 172.9265 124.90093) (width 1) (layer "F.Cu") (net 11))
 (segment (start 157.6324 128.4224) (end 144.8308 128.4224) (width 1) (layer "F.Cu") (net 11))
 (segment (start 146.939 117.635586) (end 147.839014 118.5356) (width 0.6) (layer "F.Cu") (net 11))
 (segment (start 168.722 107.8448) (end 156.874 107.8448) (width 1) (layer "F.Cu") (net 11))
 (segment (start 170.4265 113.3505) (end 170.4265 109.5493) (width 1) (layer "F.Cu") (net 11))
 (segment (start 155.5796 113.47403) (end 155.5796 112.8206) (width 1) (layer "F.Cu") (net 11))
 (segment (start 172.9265 124.90093) (end 169.40503 128.4224) (width 1) (layer "F.Cu") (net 11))
 (segment (start 146.3548 128.4224) (end 144.334694 128.4224) (width 1) (layer "F.Cu") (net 11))
 (segment (start 170.402 109.5248) (end 168.722 107.8448) (width 1) (layer "F.Cu") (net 11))
 (segment (start 144.334694 128.4224) (end 140.005 124.092706) (width 1) (layer "F.Cu") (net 11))
 (segment (start 156.874 107.8448) (end 155.5796 109.1392) (width 1) (layer "F.Cu") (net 11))
 (segment (start 155.5796 113.47403) (end 155.559 113.49463) (width 1) (layer "F.Cu") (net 11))
 (segment (start 146.939 116.524) (end 146.939 112.9781) (width 0.6) (layer "F.Cu") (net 11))
 (segment (start 152.019 116.524) (end 152.019 118.5102) (width 0.6) (layer "F.Cu") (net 11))
 (segment (start 151.9936 118.5356) (end 148.6916 118.5356) (width 1) (layer "F.Cu") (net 11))
 (segment (start 155.559 117.91107) (end 155.559 113.49463) (width 1) (layer "F.Cu") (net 11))
 (segment (start 146.939 112.9781) (end 147.5475 112.3696) (width 0.6) (layer "F.Cu") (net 11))
 (segment (start 170.4265 109.5493) (end 170.402 109.5248) (width 1) (layer "F.Cu") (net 11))
 (segment (start 154.93447 118.5356) (end 155.559 117.91107) (width 1) (layer "F.Cu") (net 11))
 (segment (start 147.839014 118.5356) (end 148.6916 118.5356) (width 0.6) (layer "F.Cu") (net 11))
 (segment (start 140.005 124.092706) (end 140.005 122.936) (width 1) (layer "F.Cu") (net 11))
 (segment (start 151.9936 118.5356) (end 154.93447 118.5356) (width 1) (layer "F.Cu") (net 11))
 (segment (start 146.939 116.524) (end 146.939 117.635586) (width 0.6) (layer "F.Cu") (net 11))
 (segment (start 152.019 118.5102) (end 151.9936 118.5356) (width 0.6) (layer "F.Cu") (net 11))
 (segment (start 155.5796 109.1392) (end 155.5796 113.47403) (width 1) (layer "F.Cu") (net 11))
 (segment (start 148.209 121.474) (end 148.209 124.3065) (width 0.6) (layer "F.Cu") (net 3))
 (segment (start 148.209 124.3065) (end 147.8015 124.714) (width 0.6) (layer "F.Cu") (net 3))
 (segment (start 145.669 121.474) (end 145.669 124.3065) (width 0.6) (layer "F.Cu") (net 1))
 (segment (start 145.669 124.3065) (end 146.0765 124.714) (width 0.6) (layer "F.Cu") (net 1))
 (segment (start 149.479 124.5605) (end 149.7595 124.841) (width 0.6) (layer "F.Cu") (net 4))
 (segment (start 149.479 121.474) (end 149.479 124.5605) (width 0.6) (layer "F.Cu") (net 4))
 (segment (start 150.749 124.1055) (end 151.4845 124.841) (width 0.6) (layer "F.Cu") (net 5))
 (segment (start 150.749 121.474) (end 150.749 124.1055) (width 0.6) (layer "F.Cu") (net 5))
 (segment (start 143.1036 124.8675) (end 143.1058 124.8653) (width 0.6) (layer "F.Cu") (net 2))
 (segment (start 145.177 119.999) (end 143.1036 122.0724) (width 0.6) (layer "F.Cu") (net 2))
 (segment (start 143.1058 124.8653) (end 143.1058 124.2557) (width 0.6) (layer "F.Cu") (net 2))
 (segment (start 143.1036 122.0724) (end 143.1036 124.8675) (width 0.6) (layer "F.Cu") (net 2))
 (segment (start 146.939 120.499001) (end 146.438999 119.999) (width 0.6) (layer "F.Cu") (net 2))
 (segment (start 146.438999 119.999) (end 145.177 119.999) (width 0.6) (layer "F.Cu") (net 2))
 (segment (start 146.939 121.474) (end 146.939 120.499001) (width 0.6) (layer "F.Cu") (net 2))
 (segment (start 153.924 125.3225) (end 153.924 126.4423) (width 0.6) (layer "F.Cu") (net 6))
 (segment (start 152.019 123.4175) (end 153.924 125.3225) (width 0.6) (layer "F.Cu") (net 6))
 (segment (start 152.019 121.474) (end 152.019 123.4175) (width 0.6) (layer "F.Cu") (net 6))
 (segment (start 127.9155 114.554) (end 127.381 115.0885) (width 0.8) (layer "F.Cu") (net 16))
 (segment (start 130.8 109.455) (end 130.8 114.132) (width 0.8) (layer "F.Cu") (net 16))
 (segment (start 130.378 114.554) (end 127.9155 114.554) (width 0.8) (layer "F.Cu") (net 16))
 (segment (start 130.8 114.132) (end 130.378 114.554) (width 0.8) (layer "F.Cu") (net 16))
 (segment (start 126.8465 116.8135) (end 127.381 116.8135) (width 0.8) (layer "F.Cu") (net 17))
 (segment (start 126.238 116.205) (end 126.8465 116.8135) (width 0.8) (layer "F.Cu") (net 17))
 (segment (start 130.378 120.269) (end 130.505 120.396) (width 0.6) (layer "F.Cu") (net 17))
 (segment (start 130.378 117.094) (end 130.378 120.269) (width 0.8) (layer "F.Cu") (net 17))
 (segment (start 127.6615 117.094) (end 127.381 116.8135) (width 0.8) (layer "F.Cu") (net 17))
 (segment (start 127.1714 109.455) (end 126.238 110.3884) (width 0.8) (layer "F.Cu") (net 17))
 (segment (start 130.378 117.094) (end 127.6615 117.094) (width 0.8) (layer "F.Cu") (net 17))
 (segment (start 126.238 110.3884) (end 126.238 116.205) (width 0.8) (layer "F.Cu") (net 17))
 (segment (start 128.26 109.455) (end 127.1714 109.455) (width 0.8) (layer "F.Cu") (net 17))
 (segment (start 157.15527 127.4224) (end 166.8546 127.4224) (width 0.6) (layer "F.Cu") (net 7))
 (segment (start 153.289 121.474) (end 153.289 123.55613) (width 0.6) (layer "F.Cu") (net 7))
 (segment (start 166.8546 127.4224) (end 170.4265 123.8505) (width 0.6) (layer "F.Cu") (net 7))
 (segment (start 153.289 123.55613) (end 157.15527 127.4224) (width 0.6) (layer "F.Cu") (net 7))
 (segment (start 168.1265 122.609712) (end 170.4265 120.309712) (width 0.6) (layer "F.Cu") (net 8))
 (segment (start 168.1265 124.544888) (end 168.1265 122.609712) (width 0.6) (layer "F.Cu") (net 8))
 (segment (start 154.559 121.474) (end 154.559 123.50643) (width 0.6) (layer "F.Cu") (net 8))
 (segment (start 157.67497 126.6224) (end 166.048988 126.6224) (width 0.6) (layer "F.Cu") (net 8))
 (segment (start 154.559 123.50643) (end 157.67497 126.6224) (width 0.6) (layer "F.Cu") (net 8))
 (segment (start 166.048988 126.6224) (end 168.1265 124.544888) (width 0.6) (layer "F.Cu") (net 8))
 (segment (start 170.4265 120.309712) (end 170.4265 120.0773) (width 0.6) (layer "F.Cu") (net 8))
 (segment (start 170.4265 120.5051) (end 170.4265 120.3505) (width 0.6) (layer "F.Cu") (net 8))
 (segment (start 127.3556 124.0376) (end 127.3556 126.3206) (width 0.8) (layer "F.Cu") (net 18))
 (segment (start 127.3556 126.3206) (end 128.27 127.235) (width 0.8) (layer "F.Cu") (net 18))
 (segment (start 131.655 116.321) (end 131.655 126.39) (width 0.6) (layer "F.Cu") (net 22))
 (segment (start 131.655 126.39) (end 130.81 127.235) (width 0.6) (layer "F.Cu") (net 22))
 (segment (start 131.158 115.824) (end 131.655 116.321) (width 0.6) (layer "F.Cu") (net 22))
 (segment (start 130.378 115.824) (end 131.158 115.824) (width 0.6) (layer "F.Cu") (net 22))
 (segment (start 150.971175 111.315175) (end 143.142025 111.315175) (width 0.6) (layer "F.Cu") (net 15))
 (segment (start 139.9032 114.554) (end 139.878 114.554) (width 0.6) (layer "F.Cu") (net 15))
 (segment (start 152.2796 112.6236) (end 150.971175 111.315175) (width 0.6) (layer "F.Cu") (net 15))
 (segment (start 143.142025 111.315175) (end 139.9032 114.554) (width 0.6) (layer "F.Cu") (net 15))
 (segment (start 154.559 116.524) (end 154.559 112.903) (width 0.6) (layer "F.Cu") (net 9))
 (segment (start 154.559 112.903) (end 154.2796 112.6236) (width 0.6) (layer "F.Cu") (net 9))
 (segment (start 128.254 122.936) (end 127.3556 122.0376) (width 0.8) (layer "F.Cu") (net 19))
 (segment (start 130.505 122.936) (end 128.254 122.936) (width 0.8) (layer "F.Cu") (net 19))
 (segment (start 138.955 113.8258) (end 142.2208 110.56) (width 0.4) (layer "F.Cu") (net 10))
 (segment (start 140.005 121.666) (end 139.446 121.666) (width 0.4) (layer "F.Cu") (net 10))
 (segment (start 139.446 121.666) (end 138.955 121.175) (width 0.4) (layer "F.Cu") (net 10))
 (segment (start 153.2796 111.8776) (end 153.2796 116.5146) (width 0.4) (layer "F.Cu") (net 10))
 (segment (start 142.2208 110.56) (end 151.962 110.56) (width 0.4) (layer "F.Cu") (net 10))
 (segment (start 151.962 110.56) (end 152.019 110.617) (width 0.4) (layer "F.Cu") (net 10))
 (segment (start 138.955 121.175) (end 138.955 113.8258) (width 0.4) (layer "F.Cu") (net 10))
 (segment (start 151.962 110.56) (end 153.2796 111.8776) (width 0.4) (layer "F.Cu") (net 10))
 (segment (start 153.2796 116.5146) (end 153.289 116.524) (width 0.4) (layer "F.Cu") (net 10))
 (segment (start 148.209 116.524) (end 149.479 116.524) (width 0.6) (layer "F.Cu") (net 13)))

